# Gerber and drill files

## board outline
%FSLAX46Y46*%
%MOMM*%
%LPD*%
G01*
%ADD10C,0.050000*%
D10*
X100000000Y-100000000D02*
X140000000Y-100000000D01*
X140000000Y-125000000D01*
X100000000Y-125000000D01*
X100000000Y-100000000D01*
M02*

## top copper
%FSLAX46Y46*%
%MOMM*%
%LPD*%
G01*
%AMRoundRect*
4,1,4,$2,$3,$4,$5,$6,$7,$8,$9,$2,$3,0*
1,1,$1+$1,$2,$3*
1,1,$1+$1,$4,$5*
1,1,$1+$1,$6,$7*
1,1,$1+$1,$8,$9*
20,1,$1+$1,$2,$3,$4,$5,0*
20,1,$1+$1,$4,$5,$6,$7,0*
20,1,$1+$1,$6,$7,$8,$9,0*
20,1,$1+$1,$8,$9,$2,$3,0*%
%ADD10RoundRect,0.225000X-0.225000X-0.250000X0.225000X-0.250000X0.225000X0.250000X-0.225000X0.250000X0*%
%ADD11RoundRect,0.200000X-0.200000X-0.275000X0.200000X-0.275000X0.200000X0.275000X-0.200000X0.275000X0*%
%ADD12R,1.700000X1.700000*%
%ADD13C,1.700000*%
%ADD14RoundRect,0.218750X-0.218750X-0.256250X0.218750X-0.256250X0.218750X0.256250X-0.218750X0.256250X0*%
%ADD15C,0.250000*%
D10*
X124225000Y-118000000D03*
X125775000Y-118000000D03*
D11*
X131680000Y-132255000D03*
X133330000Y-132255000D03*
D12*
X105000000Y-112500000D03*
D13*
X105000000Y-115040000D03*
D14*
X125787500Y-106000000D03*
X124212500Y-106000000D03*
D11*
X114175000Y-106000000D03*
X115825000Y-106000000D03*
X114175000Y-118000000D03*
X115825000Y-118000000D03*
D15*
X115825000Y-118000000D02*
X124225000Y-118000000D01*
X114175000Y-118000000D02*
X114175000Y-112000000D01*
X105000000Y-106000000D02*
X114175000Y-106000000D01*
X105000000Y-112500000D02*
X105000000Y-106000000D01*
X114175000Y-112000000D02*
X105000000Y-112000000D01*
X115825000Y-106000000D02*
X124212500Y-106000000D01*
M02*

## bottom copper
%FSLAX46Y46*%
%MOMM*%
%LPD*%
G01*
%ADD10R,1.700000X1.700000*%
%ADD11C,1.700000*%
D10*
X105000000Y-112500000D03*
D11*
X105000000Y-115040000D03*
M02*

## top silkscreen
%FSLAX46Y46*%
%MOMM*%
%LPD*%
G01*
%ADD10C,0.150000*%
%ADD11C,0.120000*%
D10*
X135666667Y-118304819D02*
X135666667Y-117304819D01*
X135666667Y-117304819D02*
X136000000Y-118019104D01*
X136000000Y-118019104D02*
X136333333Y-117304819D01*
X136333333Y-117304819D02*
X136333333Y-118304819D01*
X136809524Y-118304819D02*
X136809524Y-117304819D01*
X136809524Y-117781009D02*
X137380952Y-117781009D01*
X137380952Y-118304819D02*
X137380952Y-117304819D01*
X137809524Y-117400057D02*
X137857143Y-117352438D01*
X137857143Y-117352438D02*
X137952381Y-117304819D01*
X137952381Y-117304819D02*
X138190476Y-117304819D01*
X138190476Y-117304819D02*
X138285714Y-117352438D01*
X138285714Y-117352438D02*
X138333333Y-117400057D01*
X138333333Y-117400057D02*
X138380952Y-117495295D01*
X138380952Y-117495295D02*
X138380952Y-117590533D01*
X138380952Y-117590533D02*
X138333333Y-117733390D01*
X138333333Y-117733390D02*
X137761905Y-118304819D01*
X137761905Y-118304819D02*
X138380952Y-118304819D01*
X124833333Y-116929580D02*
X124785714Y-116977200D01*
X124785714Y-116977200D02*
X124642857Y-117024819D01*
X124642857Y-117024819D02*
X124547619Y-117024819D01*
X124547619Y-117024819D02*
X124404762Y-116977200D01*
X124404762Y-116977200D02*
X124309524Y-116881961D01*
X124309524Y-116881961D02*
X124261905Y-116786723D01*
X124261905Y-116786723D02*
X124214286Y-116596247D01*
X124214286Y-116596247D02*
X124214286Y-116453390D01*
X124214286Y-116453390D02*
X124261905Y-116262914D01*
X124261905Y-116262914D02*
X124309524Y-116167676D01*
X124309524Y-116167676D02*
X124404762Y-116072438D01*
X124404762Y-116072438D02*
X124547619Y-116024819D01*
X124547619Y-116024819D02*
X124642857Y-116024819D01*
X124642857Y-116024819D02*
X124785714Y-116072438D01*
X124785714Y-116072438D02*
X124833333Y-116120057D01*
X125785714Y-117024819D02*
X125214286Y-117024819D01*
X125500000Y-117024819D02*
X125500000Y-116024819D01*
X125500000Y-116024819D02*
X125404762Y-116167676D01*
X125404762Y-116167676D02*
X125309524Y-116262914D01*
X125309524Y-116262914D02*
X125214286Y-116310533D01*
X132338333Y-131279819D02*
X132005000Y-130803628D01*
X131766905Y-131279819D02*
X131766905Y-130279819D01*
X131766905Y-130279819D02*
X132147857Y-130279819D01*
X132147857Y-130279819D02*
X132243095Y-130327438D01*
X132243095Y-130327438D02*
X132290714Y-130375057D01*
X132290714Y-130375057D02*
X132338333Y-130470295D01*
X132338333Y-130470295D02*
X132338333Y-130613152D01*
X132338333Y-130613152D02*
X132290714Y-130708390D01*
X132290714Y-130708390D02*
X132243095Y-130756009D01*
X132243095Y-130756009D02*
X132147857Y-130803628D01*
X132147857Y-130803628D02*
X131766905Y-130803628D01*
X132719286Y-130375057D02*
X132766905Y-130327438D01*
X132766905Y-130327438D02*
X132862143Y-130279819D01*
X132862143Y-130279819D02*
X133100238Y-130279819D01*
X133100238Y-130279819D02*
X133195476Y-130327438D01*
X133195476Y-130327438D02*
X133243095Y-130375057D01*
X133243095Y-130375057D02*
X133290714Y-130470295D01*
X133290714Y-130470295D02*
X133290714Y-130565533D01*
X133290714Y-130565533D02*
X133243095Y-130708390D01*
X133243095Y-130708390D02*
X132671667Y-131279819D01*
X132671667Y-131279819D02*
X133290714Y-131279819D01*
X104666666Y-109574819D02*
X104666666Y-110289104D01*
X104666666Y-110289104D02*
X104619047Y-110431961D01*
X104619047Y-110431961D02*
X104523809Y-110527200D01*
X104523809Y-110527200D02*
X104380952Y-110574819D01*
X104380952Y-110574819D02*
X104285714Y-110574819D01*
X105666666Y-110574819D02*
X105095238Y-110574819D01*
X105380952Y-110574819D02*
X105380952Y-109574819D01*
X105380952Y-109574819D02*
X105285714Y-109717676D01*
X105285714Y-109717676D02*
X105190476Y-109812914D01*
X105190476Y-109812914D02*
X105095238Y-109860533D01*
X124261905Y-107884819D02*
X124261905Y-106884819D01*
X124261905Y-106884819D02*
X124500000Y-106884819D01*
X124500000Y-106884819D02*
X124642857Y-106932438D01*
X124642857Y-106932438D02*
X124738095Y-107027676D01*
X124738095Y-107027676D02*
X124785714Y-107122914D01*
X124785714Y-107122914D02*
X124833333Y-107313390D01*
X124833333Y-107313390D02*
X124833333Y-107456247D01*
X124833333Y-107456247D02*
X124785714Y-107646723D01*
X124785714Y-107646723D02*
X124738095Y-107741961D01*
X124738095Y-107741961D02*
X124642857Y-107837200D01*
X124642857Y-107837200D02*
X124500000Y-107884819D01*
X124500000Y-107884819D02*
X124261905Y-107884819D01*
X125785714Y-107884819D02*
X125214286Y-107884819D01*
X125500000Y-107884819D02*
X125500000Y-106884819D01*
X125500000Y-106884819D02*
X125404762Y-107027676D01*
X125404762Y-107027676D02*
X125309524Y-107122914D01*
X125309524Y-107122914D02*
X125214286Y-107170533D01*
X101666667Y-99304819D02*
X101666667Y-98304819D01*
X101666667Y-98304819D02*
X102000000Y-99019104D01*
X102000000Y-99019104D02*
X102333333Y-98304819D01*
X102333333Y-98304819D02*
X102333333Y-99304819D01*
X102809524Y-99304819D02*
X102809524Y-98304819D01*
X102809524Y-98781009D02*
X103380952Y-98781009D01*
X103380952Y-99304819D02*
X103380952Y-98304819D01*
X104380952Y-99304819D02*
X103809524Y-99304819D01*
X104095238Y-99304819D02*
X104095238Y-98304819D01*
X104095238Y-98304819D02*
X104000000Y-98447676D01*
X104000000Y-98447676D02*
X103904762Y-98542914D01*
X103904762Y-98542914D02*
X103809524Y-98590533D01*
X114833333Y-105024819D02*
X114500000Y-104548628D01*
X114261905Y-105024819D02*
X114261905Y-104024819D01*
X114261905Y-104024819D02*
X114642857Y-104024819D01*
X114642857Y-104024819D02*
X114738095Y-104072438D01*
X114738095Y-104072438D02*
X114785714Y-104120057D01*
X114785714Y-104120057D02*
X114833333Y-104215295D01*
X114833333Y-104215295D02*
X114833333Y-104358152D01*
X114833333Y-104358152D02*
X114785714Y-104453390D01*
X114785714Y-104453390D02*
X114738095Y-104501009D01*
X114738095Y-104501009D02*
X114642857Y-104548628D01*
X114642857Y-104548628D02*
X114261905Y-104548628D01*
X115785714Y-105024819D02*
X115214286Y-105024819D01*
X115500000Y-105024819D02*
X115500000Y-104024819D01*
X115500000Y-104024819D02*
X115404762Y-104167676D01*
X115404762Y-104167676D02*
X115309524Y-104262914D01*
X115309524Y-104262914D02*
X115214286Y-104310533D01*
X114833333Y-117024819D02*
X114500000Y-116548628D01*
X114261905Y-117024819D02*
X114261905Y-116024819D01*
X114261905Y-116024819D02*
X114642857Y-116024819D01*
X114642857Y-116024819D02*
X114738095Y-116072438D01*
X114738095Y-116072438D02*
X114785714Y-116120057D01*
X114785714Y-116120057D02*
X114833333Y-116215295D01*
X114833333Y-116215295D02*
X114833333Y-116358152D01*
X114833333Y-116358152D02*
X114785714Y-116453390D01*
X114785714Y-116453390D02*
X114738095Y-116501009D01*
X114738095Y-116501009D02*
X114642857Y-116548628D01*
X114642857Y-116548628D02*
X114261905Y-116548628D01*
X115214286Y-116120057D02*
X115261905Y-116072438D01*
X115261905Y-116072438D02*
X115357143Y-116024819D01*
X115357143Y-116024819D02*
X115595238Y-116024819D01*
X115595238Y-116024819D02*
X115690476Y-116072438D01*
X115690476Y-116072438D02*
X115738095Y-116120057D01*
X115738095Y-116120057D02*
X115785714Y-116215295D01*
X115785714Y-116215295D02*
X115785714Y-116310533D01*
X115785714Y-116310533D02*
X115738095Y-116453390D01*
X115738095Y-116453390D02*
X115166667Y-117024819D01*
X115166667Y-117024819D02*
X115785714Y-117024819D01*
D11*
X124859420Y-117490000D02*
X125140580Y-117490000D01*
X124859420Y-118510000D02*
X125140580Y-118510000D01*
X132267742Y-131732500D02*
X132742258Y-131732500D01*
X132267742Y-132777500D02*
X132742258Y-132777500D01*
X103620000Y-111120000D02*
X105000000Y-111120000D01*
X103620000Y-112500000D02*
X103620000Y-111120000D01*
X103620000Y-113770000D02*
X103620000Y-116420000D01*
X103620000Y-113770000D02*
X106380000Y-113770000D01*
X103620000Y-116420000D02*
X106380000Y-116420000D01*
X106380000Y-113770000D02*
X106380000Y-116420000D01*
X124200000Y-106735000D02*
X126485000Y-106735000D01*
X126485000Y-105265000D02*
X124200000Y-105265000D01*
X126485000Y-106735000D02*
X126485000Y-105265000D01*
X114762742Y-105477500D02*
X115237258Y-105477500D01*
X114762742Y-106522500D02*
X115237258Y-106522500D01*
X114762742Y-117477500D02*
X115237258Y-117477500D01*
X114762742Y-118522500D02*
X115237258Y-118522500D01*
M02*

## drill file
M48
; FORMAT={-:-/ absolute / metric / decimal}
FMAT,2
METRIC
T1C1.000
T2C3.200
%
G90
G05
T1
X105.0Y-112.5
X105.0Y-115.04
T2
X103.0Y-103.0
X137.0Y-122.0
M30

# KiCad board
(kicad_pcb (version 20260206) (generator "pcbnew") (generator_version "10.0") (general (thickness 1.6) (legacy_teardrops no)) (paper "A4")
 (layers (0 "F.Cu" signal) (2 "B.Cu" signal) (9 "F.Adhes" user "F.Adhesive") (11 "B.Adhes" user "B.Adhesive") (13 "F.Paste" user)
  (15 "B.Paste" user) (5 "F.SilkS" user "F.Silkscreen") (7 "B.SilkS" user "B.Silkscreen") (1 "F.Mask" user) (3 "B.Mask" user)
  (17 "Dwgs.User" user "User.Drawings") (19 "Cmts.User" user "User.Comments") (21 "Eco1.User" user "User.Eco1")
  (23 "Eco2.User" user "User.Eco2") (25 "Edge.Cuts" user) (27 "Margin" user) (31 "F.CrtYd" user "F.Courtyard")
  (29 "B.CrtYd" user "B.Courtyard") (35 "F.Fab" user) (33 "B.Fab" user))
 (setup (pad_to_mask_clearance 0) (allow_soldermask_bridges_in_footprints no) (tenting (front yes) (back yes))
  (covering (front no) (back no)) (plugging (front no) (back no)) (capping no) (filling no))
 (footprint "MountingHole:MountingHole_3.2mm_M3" (layer "F.Cu") (at 137 122)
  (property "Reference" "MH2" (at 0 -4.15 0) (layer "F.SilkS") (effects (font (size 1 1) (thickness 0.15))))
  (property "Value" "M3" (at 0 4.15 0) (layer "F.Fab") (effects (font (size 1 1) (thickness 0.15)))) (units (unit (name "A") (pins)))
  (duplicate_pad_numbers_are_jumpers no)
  (pad "" np_thru_hole circle (at 0 0) (size 3.2 3.2) (drill 3.2) (layers "*.Cu" "*.Mask")))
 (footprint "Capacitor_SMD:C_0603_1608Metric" (layer "F.Cu") (at 125 118)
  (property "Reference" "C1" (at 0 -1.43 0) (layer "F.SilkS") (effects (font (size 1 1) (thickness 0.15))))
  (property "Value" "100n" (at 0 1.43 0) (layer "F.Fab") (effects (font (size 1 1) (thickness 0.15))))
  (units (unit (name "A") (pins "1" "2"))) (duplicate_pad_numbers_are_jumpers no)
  (fp_line (start -0.14058 -0.51) (end 0.14058 -0.51) (stroke (width 0.12) (type solid)) (layer "F.SilkS"))
  (fp_line (start -0.14058 0.51) (end 0.14058 0.51) (stroke (width 0.12) (type solid)) (layer "F.SilkS"))
  (pad "1" smd roundrect (at -0.775 0) (size 0.9 0.95) (layers "F.Cu" "F.Mask" "F.Paste") (roundrect_rratio 0.25) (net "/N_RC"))
  (pad "2" smd roundrect (at 0.775 0) (size 0.9 0.95) (layers "F.Cu" "F.Mask" "F.Paste") (roundrect_rratio 0.25) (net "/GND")))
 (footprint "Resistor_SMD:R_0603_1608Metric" (layer "F.Cu") (at 132.505 132.255)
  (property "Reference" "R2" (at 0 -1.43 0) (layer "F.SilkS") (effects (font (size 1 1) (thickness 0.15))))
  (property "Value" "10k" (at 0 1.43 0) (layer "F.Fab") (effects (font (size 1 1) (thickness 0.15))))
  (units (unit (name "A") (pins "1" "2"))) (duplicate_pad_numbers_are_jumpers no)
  (fp_line (start -0.237258 -0.5225) (end 0.237258 -0.5225) (stroke (width 0.12) (type solid)) (layer "F.SilkS"))
  (fp_line (start -0.237258 0.5225) (end 0.237258 0.5225) (stroke (width 0.12) (type solid)) (layer "F.SilkS"))
  (pad "1" smd roundrect (at -0.825 0) (size 0.8 0.95) (layers "F.Cu" "F.Mask" "F.Paste") (roundrect_rratio 0.25) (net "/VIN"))
  (pad "2" smd roundrect (at 0.825 0) (size 0.8 0.95) (layers "F.Cu" "F.Mask" "F.Paste") (roundrect_rratio 0.25) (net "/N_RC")))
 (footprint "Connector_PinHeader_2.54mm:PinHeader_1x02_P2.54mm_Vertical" (layer "F.Cu") (at 105 112.5)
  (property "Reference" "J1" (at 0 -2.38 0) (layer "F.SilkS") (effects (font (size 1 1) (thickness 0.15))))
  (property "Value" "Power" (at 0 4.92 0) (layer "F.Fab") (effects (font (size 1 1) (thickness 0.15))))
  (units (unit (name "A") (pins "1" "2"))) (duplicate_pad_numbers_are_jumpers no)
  (fp_line (start -1.38 -1.38) (end 0 -1.38) (stroke (width 0.12) (type solid)) (layer "F.SilkS"))
  (fp_line (start -1.38 0) (end -1.38 -1.38) (stroke (width 0.12) (type solid)) (layer "F.SilkS"))
  (fp_line (start -1.38 1.27) (end -1.38 3.92) (stroke (width 0.12) (type solid)) (layer "F.SilkS"))
  (fp_line (start -1.38 1.27) (end 1.38 1.27) (stroke (width 0.12) (type solid)) (layer "F.SilkS"))
  (fp_line (start -1.38 3.92) (end 1.38 3.92) (stroke (width 0.12) (type solid)) (layer "F.SilkS"))
  (fp_line (start 1.38 1.27) (end 1.38 3.92) (stroke (width 0.12) (type solid)) (layer "F.SilkS"))
  (pad "1" thru_hole rect (at 0 0) (size 1.7 1.7) (drill 1) (layers "*.Cu" "*.Mask") (remove_unused_layers no) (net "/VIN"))
  (pad "2" thru_hole circle (at 0 2.54) (size 1.7 1.7) (drill 1) (layers "*.Cu" "*.Mask") (remove_unused_layers no) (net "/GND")))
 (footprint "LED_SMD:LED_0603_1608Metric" (layer "F.Cu") (at 125 106 180)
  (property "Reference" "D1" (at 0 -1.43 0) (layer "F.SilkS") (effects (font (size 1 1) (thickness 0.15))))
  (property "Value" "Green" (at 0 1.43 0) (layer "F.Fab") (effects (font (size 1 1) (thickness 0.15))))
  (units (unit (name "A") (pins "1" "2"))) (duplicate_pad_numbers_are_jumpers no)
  (fp_line (start 0.8 -0.735) (end -1.485 -0.735) (stroke (width 0.12) (type solid)) (layer "F.SilkS"))
  (fp_line (start -1.485 0.735) (end 0.8 0.735) (stroke (width 0.12) (type solid)) (layer "F.SilkS"))
  (fp_line (start -1.485 -0.735) (end -1.485 0.735) (stroke (width 0.12) (type solid)) (layer "F.SilkS"))
  (pad "1" smd roundrect (at -0.7875 0) (size 0.875 0.95) (layers "F.Cu" "F.Mask" "F.Paste") (roundrect_rratio 0.25) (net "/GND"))
  (pad "2" smd roundrect (at 0.7875 0) (size 0.875 0.95) (layers "F.Cu" "F.Mask" "F.Paste") (roundrect_rratio 0.25) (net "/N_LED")))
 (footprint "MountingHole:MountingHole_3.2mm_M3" (layer "F.Cu") (at 103 103)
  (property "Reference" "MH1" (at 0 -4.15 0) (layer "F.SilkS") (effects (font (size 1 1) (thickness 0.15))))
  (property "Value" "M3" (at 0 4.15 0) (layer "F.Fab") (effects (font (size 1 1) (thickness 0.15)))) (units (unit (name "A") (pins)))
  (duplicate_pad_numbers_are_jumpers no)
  (pad "" np_thru_hole circle (at 0 0) (size 3.2 3.2) (drill 3.2) (layers "*.Cu" "*.Mask")))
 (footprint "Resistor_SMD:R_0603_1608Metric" (layer "F.Cu") (at 115 106)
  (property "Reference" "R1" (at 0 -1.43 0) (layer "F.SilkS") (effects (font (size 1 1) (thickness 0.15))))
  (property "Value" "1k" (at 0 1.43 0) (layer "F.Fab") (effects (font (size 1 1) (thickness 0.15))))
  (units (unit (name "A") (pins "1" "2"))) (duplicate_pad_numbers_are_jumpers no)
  (fp_line (start -0.237258 -0.5225) (end 0.237258 -0.5225) (stroke (width 0.12) (type solid)) (layer "F.SilkS"))
  (fp_line (start -0.237258 0.5225) (end 0.237258 0.5225) (stroke (width 0.12) (type solid)) (layer "F.SilkS"))
  (pad "1" smd roundrect (at -0.825 0) (size 0.8 0.95) (layers "F.Cu" "F.Mask" "F.Paste") (roundrect_rratio 0.25) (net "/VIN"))
  (pad "2" smd roundrect (at 0.825 0) (size 0.8 0.95) (layers "F.Cu" "F.Mask" "F.Paste") (roundrect_rratio 0.25) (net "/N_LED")))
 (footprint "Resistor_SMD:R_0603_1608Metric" (layer "F.Cu") (at 115 118)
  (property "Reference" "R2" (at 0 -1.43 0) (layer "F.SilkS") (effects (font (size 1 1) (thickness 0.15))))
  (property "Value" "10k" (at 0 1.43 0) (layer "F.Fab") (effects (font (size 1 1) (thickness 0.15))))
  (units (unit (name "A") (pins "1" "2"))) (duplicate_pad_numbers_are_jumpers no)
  (fp_line (start -0.237258 -0.5225) (end 0.237258 -0.5225) (stroke (width 0.12) (type solid)) (layer "F.SilkS"))
  (fp_line (start -0.237258 0.5225) (end 0.237258 0.5225) (stroke (width 0.12) (type solid)) (layer "F.SilkS"))
  (pad "1" smd roundrect (at -0.825 0) (size 0.8 0.95) (layers "F.Cu" "F.Mask" "F.Paste") (roundrect_rratio 0.25) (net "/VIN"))
  (pad "2" smd roundrect (at 0.825 0) (size 0.8 0.95) (layers "F.Cu" "F.Mask" "F.Paste") (roundrect_rratio 0.25) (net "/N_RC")))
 (gr_rect (start 100 100) (end 140 125) (stroke (width 0.05) (type default)) (fill no) (layer "Edge.Cuts"))
 (segment (start 115.825 118) (end 124.225 118) (width 0.25) (layer "F.Cu") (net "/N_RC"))
 (segment (start 114.175 118) (end 114.175 112) (width 0.25) (layer "F.Cu") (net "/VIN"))
 (segment (start 105 106) (end 114.175 106) (width 0.25) (layer "F.Cu") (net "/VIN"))
 (segment (start 105 112.5) (end 105 106) (width 0.25) (layer "F.Cu") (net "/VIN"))
 (segment (start 114.175 112) (end 105 112) (width 0.25) (layer "F.Cu") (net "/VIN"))
 (segment (start 115.825 106) (end 124.2125 106) (width 0.25) (layer "F.Cu") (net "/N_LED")))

